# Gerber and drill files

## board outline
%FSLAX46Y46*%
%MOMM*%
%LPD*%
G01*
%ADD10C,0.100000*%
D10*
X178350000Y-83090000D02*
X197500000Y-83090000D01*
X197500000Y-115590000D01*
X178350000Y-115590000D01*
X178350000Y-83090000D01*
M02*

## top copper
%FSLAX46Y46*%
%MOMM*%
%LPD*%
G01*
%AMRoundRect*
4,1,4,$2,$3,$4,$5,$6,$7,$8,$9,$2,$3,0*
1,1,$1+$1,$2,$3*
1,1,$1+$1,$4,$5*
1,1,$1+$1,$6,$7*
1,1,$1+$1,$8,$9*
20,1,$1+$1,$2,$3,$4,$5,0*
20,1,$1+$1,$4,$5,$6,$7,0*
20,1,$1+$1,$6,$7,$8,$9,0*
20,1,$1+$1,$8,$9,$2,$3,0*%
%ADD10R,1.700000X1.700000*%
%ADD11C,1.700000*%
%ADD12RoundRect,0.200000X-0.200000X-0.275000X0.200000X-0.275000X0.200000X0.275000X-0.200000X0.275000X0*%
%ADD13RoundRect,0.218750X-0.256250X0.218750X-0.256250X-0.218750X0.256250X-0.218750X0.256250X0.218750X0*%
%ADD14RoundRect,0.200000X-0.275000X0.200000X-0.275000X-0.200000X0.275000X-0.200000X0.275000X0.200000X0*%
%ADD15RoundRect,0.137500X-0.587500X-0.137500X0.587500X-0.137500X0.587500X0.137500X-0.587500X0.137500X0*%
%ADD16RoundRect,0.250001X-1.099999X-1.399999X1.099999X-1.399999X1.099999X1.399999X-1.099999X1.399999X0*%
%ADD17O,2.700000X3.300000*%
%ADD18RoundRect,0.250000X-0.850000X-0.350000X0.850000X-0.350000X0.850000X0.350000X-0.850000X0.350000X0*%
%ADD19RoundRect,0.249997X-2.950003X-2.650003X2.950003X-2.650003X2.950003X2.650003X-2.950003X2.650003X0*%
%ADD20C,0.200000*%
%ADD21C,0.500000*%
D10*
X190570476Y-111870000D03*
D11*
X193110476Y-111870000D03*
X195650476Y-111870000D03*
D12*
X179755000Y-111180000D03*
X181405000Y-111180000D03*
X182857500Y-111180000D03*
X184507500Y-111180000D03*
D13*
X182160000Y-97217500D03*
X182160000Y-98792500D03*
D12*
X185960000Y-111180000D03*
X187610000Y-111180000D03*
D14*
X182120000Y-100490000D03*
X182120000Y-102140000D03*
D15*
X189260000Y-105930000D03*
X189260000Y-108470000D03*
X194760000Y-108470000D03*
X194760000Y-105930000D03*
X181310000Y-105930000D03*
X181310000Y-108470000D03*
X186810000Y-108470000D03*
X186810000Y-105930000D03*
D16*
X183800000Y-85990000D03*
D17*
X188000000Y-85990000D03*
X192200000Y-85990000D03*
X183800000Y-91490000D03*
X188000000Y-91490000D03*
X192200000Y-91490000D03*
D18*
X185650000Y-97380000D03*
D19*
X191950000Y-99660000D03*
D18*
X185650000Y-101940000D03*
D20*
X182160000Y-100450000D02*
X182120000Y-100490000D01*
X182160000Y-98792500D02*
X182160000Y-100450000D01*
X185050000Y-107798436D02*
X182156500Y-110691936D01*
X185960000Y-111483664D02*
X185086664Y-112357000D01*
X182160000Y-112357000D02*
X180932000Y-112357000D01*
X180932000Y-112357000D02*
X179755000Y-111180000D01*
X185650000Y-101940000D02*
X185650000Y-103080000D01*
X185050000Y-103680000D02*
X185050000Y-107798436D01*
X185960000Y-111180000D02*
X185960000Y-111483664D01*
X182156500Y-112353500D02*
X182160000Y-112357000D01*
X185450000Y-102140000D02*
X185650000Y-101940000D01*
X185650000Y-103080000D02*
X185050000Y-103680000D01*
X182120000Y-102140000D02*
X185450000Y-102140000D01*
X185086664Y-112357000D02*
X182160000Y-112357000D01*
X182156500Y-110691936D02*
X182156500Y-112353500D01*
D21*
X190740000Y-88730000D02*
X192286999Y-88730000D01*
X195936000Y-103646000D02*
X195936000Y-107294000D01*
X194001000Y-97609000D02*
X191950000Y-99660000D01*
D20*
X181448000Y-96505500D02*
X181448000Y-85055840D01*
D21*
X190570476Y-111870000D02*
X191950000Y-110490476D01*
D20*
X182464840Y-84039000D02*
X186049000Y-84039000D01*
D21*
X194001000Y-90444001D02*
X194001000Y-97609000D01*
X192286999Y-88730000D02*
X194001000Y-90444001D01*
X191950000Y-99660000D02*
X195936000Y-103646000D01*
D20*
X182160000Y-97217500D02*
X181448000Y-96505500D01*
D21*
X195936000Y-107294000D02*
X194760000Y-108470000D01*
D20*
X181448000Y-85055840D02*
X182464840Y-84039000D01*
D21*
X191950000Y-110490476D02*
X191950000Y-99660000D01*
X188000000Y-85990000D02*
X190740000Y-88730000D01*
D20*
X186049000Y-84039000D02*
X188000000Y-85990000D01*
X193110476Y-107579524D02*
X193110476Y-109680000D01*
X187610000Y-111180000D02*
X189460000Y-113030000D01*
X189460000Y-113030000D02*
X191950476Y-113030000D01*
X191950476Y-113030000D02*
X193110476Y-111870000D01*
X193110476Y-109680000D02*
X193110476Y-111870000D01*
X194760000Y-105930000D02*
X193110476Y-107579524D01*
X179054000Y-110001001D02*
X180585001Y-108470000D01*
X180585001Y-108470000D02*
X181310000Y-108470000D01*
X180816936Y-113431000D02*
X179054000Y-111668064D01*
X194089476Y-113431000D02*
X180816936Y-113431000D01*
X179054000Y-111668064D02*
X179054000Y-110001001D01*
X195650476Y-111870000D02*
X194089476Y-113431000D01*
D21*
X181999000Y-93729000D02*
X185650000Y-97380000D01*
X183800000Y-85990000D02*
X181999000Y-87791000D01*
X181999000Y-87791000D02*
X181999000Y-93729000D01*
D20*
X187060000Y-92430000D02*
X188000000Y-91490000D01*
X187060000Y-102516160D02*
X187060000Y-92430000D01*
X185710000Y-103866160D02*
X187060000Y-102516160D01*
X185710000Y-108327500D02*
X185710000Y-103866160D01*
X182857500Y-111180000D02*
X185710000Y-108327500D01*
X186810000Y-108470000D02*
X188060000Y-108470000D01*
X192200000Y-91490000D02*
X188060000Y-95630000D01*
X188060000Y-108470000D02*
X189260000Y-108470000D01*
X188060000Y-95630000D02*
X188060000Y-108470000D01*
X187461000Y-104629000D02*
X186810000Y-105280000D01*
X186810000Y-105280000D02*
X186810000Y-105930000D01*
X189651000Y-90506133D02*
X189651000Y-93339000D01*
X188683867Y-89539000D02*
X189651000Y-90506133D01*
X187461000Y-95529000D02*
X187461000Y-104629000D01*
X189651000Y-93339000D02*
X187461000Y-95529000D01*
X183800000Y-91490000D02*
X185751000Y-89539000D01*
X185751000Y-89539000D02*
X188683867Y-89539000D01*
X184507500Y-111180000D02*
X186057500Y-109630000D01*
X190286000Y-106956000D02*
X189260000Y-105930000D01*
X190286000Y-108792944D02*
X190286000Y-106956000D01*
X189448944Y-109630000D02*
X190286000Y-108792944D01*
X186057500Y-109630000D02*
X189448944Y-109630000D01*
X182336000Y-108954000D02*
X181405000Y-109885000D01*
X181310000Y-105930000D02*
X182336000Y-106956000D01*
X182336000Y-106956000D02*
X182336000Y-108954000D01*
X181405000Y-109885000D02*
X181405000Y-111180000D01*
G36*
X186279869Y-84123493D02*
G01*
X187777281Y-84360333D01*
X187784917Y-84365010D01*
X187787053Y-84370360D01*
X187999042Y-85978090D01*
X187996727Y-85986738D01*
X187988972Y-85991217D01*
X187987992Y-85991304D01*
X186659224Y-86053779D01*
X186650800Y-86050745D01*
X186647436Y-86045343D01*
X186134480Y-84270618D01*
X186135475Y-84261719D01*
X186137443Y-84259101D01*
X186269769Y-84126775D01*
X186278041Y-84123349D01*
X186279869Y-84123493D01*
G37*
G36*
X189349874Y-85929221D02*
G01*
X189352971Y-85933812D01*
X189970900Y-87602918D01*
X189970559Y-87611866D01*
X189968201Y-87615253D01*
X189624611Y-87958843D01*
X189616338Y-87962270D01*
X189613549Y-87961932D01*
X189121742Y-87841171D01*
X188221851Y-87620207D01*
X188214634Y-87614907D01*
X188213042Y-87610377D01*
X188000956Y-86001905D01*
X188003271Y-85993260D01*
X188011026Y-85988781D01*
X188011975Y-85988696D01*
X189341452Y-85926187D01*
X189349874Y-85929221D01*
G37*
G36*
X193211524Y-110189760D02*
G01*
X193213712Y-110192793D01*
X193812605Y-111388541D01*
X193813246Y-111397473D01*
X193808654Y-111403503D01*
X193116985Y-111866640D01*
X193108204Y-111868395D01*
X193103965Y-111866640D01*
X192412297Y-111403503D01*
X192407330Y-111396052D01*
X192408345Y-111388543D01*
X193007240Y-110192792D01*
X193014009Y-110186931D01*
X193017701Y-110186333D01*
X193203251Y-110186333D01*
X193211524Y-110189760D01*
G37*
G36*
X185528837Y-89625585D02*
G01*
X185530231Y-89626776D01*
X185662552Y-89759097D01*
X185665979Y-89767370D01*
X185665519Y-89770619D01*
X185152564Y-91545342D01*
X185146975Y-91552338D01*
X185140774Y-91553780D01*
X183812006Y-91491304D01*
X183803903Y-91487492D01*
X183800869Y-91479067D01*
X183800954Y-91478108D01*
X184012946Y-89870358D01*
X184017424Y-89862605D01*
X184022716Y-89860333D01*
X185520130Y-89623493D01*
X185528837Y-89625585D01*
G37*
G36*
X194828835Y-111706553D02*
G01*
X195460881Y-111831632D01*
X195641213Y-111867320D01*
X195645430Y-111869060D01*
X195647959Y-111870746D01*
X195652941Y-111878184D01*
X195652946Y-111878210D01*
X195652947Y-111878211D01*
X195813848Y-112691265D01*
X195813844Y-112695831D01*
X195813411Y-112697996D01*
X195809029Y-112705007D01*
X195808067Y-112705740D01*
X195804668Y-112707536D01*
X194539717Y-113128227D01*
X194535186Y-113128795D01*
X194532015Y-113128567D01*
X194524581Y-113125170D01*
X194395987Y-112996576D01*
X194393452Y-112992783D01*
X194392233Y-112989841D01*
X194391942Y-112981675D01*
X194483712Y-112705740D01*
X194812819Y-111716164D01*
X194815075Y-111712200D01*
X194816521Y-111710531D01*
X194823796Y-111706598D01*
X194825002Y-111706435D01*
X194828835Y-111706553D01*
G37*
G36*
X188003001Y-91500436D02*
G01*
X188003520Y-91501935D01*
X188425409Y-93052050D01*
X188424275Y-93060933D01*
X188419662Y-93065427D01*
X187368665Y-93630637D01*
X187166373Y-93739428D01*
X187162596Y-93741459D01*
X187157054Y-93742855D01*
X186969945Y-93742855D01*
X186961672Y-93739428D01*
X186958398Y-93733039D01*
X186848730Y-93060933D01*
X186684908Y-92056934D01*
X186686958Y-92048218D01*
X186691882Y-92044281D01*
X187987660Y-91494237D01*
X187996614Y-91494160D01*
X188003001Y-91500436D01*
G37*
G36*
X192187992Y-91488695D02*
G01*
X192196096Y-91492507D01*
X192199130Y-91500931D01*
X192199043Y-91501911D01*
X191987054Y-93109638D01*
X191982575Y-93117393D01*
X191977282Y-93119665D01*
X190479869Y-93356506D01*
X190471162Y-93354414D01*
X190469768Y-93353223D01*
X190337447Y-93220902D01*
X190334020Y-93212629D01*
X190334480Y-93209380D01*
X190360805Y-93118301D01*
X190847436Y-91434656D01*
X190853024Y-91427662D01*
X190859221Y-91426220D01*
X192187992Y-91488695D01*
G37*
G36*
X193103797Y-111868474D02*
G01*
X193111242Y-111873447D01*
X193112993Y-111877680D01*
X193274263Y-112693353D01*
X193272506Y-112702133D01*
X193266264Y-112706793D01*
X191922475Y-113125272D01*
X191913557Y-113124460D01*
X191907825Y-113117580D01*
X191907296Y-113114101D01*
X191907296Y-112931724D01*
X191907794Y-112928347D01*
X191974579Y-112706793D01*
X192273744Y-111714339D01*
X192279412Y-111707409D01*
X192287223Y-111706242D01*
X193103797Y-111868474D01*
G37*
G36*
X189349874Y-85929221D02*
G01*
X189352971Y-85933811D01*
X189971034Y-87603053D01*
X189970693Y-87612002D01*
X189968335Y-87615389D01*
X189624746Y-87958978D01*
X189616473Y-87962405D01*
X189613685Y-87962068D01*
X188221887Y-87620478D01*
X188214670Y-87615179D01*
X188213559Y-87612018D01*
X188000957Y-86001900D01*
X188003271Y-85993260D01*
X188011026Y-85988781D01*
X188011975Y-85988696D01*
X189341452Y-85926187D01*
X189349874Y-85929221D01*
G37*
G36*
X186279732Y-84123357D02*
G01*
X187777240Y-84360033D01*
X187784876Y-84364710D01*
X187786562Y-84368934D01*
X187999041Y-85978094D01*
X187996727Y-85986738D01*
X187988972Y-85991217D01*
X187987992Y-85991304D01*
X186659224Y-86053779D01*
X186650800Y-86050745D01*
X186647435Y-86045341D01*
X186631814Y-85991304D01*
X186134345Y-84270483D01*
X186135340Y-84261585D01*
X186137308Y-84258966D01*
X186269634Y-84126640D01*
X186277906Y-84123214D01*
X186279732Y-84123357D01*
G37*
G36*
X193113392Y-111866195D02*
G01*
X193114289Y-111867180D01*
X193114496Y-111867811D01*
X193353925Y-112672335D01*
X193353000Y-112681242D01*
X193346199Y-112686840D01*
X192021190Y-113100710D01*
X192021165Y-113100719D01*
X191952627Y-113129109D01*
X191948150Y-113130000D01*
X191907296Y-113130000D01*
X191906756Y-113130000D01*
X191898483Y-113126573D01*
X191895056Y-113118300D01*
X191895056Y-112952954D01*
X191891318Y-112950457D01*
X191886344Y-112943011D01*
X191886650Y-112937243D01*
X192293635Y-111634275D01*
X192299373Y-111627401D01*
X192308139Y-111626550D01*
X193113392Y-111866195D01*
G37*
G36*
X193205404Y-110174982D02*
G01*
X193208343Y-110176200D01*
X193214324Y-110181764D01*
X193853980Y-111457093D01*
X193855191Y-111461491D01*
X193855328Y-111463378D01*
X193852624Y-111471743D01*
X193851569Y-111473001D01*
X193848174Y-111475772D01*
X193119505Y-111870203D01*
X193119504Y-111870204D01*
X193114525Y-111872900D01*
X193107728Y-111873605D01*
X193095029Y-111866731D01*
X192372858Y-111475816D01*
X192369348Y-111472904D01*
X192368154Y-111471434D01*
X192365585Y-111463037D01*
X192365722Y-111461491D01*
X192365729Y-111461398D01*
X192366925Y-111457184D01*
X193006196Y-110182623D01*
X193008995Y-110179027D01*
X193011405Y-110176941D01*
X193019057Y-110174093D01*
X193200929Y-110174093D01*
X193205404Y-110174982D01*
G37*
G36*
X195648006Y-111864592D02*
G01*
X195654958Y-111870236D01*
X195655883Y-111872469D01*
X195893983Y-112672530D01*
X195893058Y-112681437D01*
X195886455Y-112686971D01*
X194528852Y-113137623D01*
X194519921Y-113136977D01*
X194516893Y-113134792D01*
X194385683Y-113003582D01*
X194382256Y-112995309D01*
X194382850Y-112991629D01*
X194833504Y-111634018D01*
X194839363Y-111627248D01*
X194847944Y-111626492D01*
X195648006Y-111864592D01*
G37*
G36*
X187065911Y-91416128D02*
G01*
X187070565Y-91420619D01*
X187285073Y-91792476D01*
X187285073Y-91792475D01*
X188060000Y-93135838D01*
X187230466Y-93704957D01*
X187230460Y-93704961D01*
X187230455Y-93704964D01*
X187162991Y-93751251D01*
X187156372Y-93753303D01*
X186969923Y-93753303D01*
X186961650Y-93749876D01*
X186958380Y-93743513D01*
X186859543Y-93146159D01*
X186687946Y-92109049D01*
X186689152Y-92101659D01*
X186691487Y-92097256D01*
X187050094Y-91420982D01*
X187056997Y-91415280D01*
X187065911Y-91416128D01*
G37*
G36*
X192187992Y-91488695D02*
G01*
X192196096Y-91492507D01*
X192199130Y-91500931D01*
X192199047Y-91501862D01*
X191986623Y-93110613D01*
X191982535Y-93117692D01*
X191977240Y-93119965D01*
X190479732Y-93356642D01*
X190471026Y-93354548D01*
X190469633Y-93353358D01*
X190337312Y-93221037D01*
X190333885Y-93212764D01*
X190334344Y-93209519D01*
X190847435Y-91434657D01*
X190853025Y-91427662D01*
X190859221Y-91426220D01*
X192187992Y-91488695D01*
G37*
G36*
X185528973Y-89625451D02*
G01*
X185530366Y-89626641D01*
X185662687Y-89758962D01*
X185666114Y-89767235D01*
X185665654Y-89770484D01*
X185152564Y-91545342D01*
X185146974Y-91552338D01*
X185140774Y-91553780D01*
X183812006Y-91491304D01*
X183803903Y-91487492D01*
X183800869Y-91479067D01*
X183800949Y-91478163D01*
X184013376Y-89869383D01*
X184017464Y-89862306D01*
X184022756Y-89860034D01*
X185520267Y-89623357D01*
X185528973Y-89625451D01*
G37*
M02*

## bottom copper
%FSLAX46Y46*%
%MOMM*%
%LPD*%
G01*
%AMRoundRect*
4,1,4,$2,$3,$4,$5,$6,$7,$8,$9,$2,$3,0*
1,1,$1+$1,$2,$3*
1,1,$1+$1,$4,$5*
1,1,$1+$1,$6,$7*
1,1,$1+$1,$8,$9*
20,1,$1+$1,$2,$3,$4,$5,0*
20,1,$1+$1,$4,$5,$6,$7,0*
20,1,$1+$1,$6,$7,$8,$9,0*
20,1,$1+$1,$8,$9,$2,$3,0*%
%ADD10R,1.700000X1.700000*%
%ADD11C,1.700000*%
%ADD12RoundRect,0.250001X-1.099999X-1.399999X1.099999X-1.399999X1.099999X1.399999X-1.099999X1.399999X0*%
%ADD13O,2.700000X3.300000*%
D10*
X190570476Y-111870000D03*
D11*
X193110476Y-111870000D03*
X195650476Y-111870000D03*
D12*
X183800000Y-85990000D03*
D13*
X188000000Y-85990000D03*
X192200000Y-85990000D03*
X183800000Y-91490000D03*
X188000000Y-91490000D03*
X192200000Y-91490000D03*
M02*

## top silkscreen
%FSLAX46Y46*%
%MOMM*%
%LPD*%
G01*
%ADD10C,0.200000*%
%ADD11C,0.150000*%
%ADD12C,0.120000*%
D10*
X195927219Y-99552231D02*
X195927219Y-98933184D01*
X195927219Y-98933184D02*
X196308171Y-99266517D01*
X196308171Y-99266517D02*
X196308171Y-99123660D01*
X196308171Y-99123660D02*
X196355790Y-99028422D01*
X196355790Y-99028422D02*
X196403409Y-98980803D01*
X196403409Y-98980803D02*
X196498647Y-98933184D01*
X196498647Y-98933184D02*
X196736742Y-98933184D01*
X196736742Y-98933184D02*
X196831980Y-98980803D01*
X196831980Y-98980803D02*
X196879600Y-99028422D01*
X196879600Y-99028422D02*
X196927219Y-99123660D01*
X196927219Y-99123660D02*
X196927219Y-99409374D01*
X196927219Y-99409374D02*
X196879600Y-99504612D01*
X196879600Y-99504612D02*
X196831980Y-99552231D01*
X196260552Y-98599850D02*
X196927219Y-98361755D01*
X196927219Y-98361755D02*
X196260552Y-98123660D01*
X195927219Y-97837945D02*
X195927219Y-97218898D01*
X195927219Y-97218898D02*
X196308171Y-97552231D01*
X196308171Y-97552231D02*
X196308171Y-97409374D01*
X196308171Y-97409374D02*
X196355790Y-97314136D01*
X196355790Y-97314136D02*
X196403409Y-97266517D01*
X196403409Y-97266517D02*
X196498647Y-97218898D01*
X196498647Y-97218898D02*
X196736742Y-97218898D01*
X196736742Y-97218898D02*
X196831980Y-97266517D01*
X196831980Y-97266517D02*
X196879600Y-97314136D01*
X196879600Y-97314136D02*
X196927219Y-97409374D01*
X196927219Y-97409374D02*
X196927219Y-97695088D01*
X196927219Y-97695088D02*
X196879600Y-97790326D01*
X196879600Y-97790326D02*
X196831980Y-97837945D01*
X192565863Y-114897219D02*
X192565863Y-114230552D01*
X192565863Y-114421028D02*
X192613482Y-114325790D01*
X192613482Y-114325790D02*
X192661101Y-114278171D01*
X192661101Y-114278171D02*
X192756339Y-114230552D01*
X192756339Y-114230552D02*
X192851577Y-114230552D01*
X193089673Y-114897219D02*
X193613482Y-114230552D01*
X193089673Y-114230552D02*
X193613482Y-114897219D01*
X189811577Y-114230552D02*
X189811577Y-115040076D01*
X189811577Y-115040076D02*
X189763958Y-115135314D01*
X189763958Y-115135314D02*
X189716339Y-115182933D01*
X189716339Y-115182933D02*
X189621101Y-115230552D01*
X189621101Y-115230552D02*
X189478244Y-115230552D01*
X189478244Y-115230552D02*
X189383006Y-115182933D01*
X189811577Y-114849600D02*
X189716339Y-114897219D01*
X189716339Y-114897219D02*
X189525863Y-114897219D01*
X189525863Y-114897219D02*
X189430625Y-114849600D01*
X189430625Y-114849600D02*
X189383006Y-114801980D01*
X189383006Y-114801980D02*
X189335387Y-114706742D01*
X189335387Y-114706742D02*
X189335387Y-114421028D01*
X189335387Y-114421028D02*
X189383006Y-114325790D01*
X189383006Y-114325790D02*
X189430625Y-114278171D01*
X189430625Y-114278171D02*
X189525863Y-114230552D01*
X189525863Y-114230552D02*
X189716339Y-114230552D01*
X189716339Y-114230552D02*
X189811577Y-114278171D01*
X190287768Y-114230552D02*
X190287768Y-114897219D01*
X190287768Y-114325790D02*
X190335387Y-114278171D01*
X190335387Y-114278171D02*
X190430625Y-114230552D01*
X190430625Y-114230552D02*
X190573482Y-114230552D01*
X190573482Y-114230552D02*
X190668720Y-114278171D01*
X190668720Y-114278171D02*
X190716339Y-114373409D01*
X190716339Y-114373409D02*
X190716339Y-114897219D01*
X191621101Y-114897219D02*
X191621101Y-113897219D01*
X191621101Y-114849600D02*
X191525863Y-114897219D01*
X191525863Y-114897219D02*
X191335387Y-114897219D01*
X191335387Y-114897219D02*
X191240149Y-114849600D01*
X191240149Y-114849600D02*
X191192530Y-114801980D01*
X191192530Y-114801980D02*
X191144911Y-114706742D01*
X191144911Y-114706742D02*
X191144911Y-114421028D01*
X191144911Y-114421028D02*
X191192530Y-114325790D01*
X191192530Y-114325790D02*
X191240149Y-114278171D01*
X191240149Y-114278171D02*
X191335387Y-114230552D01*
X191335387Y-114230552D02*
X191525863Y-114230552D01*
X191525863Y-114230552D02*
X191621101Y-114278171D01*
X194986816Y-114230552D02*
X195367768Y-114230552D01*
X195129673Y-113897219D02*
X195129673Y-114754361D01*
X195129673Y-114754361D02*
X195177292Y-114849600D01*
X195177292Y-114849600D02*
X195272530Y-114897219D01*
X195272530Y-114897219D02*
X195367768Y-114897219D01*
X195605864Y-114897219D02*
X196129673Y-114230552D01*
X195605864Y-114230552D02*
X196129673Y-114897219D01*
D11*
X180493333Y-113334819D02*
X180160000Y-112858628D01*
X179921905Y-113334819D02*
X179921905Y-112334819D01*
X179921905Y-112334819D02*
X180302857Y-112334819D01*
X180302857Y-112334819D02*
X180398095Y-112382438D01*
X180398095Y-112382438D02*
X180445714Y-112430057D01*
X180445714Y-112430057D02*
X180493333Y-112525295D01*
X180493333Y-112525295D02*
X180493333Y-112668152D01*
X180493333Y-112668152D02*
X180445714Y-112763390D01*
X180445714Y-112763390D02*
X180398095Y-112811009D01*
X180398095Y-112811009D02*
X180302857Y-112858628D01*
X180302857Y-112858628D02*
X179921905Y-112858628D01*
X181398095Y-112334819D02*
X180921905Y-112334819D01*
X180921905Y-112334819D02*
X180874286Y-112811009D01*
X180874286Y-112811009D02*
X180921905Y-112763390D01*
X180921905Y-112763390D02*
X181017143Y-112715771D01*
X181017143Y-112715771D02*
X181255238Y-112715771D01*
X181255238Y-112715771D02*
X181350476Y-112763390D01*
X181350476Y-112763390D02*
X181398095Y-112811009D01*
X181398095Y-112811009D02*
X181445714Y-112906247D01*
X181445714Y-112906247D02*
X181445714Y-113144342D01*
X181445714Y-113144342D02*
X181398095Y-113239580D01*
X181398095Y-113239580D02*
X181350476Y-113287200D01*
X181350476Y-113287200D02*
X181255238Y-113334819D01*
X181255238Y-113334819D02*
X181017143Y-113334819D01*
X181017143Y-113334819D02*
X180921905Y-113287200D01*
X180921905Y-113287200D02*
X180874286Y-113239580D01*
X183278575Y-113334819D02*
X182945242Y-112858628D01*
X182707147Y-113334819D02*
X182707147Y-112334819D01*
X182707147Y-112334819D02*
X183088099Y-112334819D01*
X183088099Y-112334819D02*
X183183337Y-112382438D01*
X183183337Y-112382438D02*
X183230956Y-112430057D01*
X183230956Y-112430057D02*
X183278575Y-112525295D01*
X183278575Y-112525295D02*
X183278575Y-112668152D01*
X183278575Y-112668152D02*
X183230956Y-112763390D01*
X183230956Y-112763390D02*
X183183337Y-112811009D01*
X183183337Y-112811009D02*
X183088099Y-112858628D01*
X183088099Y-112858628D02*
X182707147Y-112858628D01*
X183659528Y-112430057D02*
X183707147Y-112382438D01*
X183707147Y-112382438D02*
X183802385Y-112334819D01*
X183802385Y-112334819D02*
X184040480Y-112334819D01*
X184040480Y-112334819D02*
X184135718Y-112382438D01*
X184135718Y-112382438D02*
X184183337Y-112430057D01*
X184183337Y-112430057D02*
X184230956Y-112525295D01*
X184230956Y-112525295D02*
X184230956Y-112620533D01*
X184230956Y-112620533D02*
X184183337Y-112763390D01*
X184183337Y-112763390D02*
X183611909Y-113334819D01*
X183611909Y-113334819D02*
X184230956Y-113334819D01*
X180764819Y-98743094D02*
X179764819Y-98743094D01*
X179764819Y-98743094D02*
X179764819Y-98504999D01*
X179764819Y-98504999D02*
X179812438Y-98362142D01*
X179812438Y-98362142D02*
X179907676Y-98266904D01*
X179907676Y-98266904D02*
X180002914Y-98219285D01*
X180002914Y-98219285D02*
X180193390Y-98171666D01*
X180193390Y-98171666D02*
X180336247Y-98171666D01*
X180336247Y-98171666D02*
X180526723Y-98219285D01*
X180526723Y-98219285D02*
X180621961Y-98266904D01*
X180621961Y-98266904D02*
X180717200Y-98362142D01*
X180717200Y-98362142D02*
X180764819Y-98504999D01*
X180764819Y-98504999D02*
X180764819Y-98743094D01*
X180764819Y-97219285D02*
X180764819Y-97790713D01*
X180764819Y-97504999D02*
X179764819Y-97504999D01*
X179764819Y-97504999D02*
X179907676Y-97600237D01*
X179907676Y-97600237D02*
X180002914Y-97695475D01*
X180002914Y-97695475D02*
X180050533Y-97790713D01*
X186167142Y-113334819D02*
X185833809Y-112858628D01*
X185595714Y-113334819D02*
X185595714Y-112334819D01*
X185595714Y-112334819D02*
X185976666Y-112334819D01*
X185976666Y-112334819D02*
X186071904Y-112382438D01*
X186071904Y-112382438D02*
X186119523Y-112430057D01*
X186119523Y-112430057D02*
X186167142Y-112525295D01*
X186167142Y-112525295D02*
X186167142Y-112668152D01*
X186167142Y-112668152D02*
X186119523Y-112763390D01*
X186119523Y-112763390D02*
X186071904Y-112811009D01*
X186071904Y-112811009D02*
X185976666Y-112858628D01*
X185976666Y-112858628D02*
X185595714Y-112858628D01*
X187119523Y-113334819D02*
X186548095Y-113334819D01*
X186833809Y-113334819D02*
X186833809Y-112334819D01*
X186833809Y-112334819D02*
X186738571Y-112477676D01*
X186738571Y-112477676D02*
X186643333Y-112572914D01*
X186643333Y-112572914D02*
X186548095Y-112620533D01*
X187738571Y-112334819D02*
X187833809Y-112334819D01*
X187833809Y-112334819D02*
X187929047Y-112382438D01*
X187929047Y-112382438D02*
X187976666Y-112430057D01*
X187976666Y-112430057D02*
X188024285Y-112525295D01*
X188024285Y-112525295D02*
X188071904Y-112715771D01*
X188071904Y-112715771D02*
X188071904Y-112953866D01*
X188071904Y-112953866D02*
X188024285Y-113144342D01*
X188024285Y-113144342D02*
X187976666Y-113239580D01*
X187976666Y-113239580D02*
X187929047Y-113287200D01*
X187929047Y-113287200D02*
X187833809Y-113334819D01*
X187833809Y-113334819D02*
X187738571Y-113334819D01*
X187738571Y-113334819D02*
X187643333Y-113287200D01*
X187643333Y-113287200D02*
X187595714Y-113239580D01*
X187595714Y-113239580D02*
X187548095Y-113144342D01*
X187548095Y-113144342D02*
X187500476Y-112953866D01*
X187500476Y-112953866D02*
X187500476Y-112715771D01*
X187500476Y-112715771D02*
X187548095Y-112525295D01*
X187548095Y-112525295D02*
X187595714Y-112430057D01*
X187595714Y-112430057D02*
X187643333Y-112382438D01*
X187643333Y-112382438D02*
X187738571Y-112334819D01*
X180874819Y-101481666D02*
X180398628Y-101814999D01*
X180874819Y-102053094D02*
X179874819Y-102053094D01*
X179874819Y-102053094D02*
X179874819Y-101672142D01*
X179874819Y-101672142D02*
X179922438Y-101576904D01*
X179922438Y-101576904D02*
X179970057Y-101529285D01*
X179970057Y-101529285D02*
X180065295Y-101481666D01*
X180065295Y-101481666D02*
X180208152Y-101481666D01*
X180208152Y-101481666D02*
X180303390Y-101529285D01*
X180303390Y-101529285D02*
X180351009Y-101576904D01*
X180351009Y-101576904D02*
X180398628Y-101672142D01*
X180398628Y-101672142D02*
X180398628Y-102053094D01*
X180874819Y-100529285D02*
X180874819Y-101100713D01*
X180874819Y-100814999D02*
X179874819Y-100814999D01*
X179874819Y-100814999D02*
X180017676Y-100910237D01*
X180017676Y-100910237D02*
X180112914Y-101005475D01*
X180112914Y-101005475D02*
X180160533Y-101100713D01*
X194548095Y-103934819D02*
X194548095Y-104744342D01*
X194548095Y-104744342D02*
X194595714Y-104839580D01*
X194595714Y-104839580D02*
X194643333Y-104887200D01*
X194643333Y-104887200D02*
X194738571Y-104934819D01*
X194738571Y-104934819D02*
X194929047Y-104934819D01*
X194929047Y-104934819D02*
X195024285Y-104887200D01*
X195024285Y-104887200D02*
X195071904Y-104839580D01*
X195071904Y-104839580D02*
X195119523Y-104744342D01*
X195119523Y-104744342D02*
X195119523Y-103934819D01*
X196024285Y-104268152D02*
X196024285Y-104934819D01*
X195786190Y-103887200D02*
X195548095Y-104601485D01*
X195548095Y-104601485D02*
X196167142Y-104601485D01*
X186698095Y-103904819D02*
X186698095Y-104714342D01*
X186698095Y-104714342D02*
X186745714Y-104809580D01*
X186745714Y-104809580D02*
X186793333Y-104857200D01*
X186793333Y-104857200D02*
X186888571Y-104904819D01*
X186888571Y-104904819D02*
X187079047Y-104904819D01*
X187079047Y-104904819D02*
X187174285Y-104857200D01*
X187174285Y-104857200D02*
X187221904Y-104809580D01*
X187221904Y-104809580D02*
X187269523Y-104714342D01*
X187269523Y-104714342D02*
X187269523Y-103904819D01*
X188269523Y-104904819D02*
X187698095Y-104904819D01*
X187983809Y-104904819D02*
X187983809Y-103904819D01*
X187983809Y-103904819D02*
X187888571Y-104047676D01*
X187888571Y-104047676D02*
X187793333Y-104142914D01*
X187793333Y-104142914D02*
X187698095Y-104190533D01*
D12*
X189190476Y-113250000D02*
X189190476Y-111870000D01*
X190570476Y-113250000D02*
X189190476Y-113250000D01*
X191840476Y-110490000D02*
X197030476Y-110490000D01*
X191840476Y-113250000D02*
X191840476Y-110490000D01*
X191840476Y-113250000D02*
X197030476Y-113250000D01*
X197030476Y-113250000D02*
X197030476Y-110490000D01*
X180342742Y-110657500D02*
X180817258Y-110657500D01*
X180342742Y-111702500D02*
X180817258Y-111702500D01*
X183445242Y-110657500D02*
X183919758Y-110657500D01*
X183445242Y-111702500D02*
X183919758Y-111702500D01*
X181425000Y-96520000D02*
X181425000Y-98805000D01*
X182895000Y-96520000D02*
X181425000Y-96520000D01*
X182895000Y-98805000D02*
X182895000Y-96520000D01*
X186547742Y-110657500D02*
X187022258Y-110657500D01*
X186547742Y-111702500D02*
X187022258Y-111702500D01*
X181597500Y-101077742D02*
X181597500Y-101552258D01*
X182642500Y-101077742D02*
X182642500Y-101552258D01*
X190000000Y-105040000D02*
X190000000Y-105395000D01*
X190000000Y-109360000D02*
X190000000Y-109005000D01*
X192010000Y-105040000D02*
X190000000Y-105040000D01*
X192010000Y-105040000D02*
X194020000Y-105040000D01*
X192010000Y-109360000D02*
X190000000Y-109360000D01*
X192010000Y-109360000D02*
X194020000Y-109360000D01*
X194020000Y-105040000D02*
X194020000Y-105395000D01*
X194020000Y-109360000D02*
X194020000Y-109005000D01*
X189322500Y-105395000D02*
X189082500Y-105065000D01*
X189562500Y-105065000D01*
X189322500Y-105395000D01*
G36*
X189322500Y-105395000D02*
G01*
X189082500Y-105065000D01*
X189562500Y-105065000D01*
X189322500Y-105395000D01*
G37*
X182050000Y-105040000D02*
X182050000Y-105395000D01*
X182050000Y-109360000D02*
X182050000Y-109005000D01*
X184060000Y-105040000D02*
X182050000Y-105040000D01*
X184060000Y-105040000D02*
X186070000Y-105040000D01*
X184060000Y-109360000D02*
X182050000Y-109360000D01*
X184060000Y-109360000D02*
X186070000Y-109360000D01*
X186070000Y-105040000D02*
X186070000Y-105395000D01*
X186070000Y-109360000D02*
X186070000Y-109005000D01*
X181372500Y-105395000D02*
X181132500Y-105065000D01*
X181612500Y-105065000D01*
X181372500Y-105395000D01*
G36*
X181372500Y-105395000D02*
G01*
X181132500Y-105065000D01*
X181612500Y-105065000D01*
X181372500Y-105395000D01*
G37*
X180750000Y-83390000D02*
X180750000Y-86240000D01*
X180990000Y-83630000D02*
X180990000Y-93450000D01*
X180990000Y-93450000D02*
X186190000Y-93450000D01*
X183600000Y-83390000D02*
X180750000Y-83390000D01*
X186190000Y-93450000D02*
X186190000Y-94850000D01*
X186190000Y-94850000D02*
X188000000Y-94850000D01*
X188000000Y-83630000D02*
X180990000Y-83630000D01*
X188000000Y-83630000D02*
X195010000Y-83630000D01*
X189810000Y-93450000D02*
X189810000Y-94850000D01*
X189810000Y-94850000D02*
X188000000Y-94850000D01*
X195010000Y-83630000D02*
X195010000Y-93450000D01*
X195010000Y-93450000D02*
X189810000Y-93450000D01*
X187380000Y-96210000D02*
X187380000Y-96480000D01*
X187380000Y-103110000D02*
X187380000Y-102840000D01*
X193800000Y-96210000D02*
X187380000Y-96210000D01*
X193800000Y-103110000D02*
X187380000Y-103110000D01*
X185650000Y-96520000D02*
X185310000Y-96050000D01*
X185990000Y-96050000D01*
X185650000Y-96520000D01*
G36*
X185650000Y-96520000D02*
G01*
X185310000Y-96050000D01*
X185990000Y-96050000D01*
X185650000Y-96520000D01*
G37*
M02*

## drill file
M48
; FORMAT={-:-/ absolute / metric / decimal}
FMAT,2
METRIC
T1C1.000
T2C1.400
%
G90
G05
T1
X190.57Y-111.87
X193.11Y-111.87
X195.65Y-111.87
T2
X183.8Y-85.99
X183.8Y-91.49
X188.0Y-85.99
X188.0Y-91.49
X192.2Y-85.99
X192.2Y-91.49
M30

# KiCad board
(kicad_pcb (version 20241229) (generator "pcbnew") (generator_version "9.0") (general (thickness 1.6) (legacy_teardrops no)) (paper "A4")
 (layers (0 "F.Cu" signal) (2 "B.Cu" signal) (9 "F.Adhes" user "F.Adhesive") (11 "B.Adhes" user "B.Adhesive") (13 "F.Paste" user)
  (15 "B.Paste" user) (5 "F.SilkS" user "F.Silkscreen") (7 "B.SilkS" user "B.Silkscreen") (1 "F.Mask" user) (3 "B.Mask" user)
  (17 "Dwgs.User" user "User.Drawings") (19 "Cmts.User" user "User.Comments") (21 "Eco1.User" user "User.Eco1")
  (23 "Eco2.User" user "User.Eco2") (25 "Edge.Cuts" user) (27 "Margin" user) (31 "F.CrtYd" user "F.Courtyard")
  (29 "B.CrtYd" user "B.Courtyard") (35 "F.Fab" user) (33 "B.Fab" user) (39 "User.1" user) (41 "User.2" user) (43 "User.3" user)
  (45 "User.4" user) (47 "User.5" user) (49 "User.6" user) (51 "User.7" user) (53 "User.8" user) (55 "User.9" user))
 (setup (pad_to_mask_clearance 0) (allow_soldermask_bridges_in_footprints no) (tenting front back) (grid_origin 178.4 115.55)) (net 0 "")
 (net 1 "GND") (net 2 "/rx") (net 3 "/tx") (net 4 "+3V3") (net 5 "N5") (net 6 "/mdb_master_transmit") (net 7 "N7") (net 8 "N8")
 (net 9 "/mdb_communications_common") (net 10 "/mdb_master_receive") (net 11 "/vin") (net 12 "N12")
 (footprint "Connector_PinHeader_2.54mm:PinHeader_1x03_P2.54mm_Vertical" (layer "F.Cu") (at 190.570476 111.87 90)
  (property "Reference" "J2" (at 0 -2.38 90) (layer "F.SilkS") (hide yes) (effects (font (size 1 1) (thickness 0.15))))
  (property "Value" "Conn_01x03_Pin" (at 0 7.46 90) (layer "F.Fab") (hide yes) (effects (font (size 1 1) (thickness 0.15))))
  (fp_line (start -1.38 -1.38) (end 0 -1.38) (stroke (width 0.12) (type solid)) (layer "F.SilkS"))
  (fp_line (start -1.38 0) (end -1.38 -1.38) (stroke (width 0.12) (type solid)) (layer "F.SilkS"))
  (fp_line (start 1.38 1.27) (end 1.38 6.46) (stroke (width 0.12) (type solid)) (layer "F.SilkS"))
  (fp_line (start -1.38 1.27) (end 1.38 1.27) (stroke (width 0.12) (type solid)) (layer "F.SilkS"))
  (fp_line (start -1.38 1.27) (end -1.38 6.46) (stroke (width 0.12) (type solid)) (layer "F.SilkS"))
  (fp_line (start -1.38 6.46) (end 1.38 6.46) (stroke (width 0.12) (type solid)) (layer "F.SilkS"))
  (pad "1" thru_hole rect (at 0 0 90) (size 1.7 1.7) (drill 1) (layers "*.Cu" "*.Mask") (remove_unused_layers no) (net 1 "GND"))
  (pad "2" thru_hole circle (at 0 2.54 90) (size 1.7 1.7) (drill 1) (layers "*.Cu" "*.Mask") (remove_unused_layers no) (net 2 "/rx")
   (teardrops (best_length_ratio 0.5) (max_length 1) (best_width_ratio 1) (max_width 2) (curved_edges no) (filter_ratio 0.9) (enabled yes)
    (allow_two_segments yes) (prefer_zone_connections yes)))
  (pad "3" thru_hole circle (at 0 5.08 90) (size 1.7 1.7) (drill 1) (layers "*.Cu" "*.Mask") (remove_unused_layers no) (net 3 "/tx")
   (teardrops (best_length_ratio 0.5) (max_length 1) (best_width_ratio 1) (max_width 2) (curved_edges no) (filter_ratio 0.9) (enabled yes)
    (allow_two_segments yes) (prefer_zone_connections yes))))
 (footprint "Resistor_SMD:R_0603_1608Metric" (layer "F.Cu") (at 180.58 111.18)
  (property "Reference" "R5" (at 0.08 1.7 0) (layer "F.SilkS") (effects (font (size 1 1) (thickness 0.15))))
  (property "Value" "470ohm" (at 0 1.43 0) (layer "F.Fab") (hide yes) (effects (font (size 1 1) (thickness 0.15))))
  (fp_line (start -0.237258 -0.5225) (end 0.237258 -0.5225) (stroke (width 0.12) (type solid)) (layer "F.SilkS"))
  (fp_line (start -0.237258 0.5225) (end 0.237258 0.5225) (stroke (width 0.12) (type solid)) (layer "F.SilkS"))
  (pad "1" smd roundrect (at -0.825 0) (size 0.8 0.95) (layers "F.Cu" "F.Mask" "F.Paste") (roundrect_rratio 0.25) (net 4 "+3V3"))
  (pad "2" smd roundrect (at 0.825 0) (size 0.8 0.95) (layers "F.Cu" "F.Mask" "F.Paste") (roundrect_rratio 0.25) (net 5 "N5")))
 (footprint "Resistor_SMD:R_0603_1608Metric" (layer "F.Cu") (at 183.6825 111.18)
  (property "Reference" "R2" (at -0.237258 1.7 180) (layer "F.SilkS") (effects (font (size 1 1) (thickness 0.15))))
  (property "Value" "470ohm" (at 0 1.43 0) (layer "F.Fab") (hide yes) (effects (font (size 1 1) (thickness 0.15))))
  (fp_line (start -0.237258 -0.5225) (end 0.237258 -0.5225) (stroke (width 0.12) (type solid)) (layer "F.SilkS"))
  (fp_line (start -0.237258 0.5225) (end 0.237258 0.5225) (stroke (width 0.12) (type solid)) (layer "F.SilkS"))
  (pad "1" smd roundrect (at -0.825 0) (size 0.8 0.95) (layers "F.Cu" "F.Mask" "F.Paste") (roundrect_rratio 0.25)
   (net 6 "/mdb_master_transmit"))
  (pad "2" smd roundrect (at 0.825 0) (size 0.8 0.95) (layers "F.Cu" "F.Mask" "F.Paste") (roundrect_rratio 0.25) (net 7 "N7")))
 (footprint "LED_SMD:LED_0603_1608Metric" (layer "F.Cu") (at 182.16 98.005 -90)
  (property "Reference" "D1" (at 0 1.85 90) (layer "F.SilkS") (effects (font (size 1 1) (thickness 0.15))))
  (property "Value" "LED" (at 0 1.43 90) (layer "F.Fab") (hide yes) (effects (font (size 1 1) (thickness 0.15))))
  (fp_line (start -1.485 0.735) (end 0.8 0.735) (stroke (width 0.12) (type solid)) (layer "F.SilkS"))
  (fp_line (start -1.485 -0.735) (end -1.485 0.735) (stroke (width 0.12) (type solid)) (layer "F.SilkS"))
  (fp_line (start 0.8 -0.735) (end -1.485 -0.735) (stroke (width 0.12) (type solid)) (layer "F.SilkS"))
  (pad "1" smd roundrect (at -0.7875 0 270) (size 0.875 0.95) (layers "F.Cu" "F.Mask" "F.Paste") (roundrect_rratio 0.25) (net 1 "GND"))
  (pad "2" smd roundrect (at 0.7875 0 270) (size 0.875 0.95) (layers "F.Cu" "F.Mask" "F.Paste") (roundrect_rratio 0.25) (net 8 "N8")))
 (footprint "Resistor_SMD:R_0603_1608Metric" (layer "F.Cu") (at 186.785 111.18)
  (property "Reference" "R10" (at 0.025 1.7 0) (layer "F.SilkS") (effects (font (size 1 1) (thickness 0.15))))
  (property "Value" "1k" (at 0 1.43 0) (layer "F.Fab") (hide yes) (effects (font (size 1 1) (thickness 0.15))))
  (fp_line (start -0.237258 -0.5225) (end 0.237258 -0.5225) (stroke (width 0.12) (type solid)) (layer "F.SilkS"))
  (fp_line (start -0.237258 0.5225) (end 0.237258 0.5225) (stroke (width 0.12) (type solid)) (layer "F.SilkS"))
  (pad "1" smd roundrect (at -0.825 0) (size 0.8 0.95) (layers "F.Cu" "F.Mask" "F.Paste") (roundrect_rratio 0.25) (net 4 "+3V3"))
  (pad "2" smd roundrect (at 0.825 0) (size 0.8 0.95) (layers "F.Cu" "F.Mask" "F.Paste") (roundrect_rratio 0.25) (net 2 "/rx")))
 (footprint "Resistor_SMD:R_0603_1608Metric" (layer "F.Cu") (at 182.12 101.315 -90)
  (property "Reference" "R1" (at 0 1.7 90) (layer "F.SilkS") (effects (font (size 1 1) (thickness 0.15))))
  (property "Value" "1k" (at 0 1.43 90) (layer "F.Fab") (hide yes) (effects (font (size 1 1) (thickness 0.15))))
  (fp_line (start -0.237258 0.5225) (end 0.237258 0.5225) (stroke (width 0.12) (type solid)) (layer "F.SilkS"))
  (fp_line (start -0.237258 -0.5225) (end 0.237258 -0.5225) (stroke (width 0.12) (type solid)) (layer "F.SilkS"))
  (pad "1" smd roundrect (at -0.825 0 270) (size 0.8 0.95) (layers "F.Cu" "F.Mask" "F.Paste") (roundrect_rratio 0.25) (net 8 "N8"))
  (pad "2" smd roundrect (at 0.825 0 270) (size 0.8 0.95) (layers "F.Cu" "F.Mask" "F.Paste") (roundrect_rratio 0.25) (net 4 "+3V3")))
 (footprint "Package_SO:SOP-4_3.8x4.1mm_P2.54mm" (layer "F.Cu") (at 192.01 107.2)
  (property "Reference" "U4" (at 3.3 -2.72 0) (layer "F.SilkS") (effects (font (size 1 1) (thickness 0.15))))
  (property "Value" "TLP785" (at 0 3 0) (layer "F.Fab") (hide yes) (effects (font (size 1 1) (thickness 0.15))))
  (fp_line (start -2.01 -2.16) (end -2.01 -1.805) (stroke (width 0.12) (type solid)) (layer "F.SilkS"))
  (fp_line (start -2.01 2.16) (end -2.01 1.805) (stroke (width 0.12) (type solid)) (layer "F.SilkS"))
  (fp_line (start 0 -2.16) (end -2.01 -2.16) (stroke (width 0.12) (type solid)) (layer "F.SilkS"))
  (fp_line (start 0 -2.16) (end 2.01 -2.16) (stroke (width 0.12) (type solid)) (layer "F.SilkS"))
  (fp_line (start 0 2.16) (end -2.01 2.16) (stroke (width 0.12) (type solid)) (layer "F.SilkS"))
  (fp_line (start 0 2.16) (end 2.01 2.16) (stroke (width 0.12) (type solid)) (layer "F.SilkS"))
  (fp_line (start 2.01 -2.16) (end 2.01 -1.805) (stroke (width 0.12) (type solid)) (layer "F.SilkS"))
  (fp_line (start 2.01 2.16) (end 2.01 1.805) (stroke (width 0.12) (type solid)) (layer "F.SilkS"))
  (fp_poly
   (pts (xy -2.6875 -1.805) (xy -2.9275 -2.135) (xy -2.4475 -2.135)) (stroke (width 0.12) (type solid)) (fill yes) (layer "F.SilkS"))
  (pad "1" smd roundrect (at -2.75 -1.27) (size 1.45 0.55) (layers "F.Cu" "F.Mask" "F.Paste") (roundrect_rratio 0.25) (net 7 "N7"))
  (pad "2" smd roundrect (at -2.75 1.27) (size 1.45 0.55) (layers "F.Cu" "F.Mask" "F.Paste") (roundrect_rratio 0.25)
   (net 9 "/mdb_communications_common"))
  (pad "3" smd roundrect (at 2.75 1.27) (size 1.45 0.55) (layers "F.Cu" "F.Mask" "F.Paste") (roundrect_rratio 0.25) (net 1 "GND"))
  (pad "4" smd roundrect (at 2.75 -1.27) (size 1.45 0.55) (layers "F.Cu" "F.Mask" "F.Paste") (roundrect_rratio 0.25) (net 2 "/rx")))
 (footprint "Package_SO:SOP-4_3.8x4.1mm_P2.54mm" (layer "F.Cu") (at 184.06 107.2)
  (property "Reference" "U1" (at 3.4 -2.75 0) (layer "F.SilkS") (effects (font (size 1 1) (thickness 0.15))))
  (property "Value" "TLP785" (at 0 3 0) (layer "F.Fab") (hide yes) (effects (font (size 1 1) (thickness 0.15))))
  (fp_line (start -2.01 -2.16) (end -2.01 -1.805) (stroke (width 0.12) (type solid)) (layer "F.SilkS"))
  (fp_line (start -2.01 2.16) (end -2.01 1.805) (stroke (width 0.12) (type solid)) (layer "F.SilkS"))
  (fp_line (start 0 -2.16) (end -2.01 -2.16) (stroke (width 0.12) (type solid)) (layer "F.SilkS"))
  (fp_line (start 0 -2.16) (end 2.01 -2.16) (stroke (width 0.12) (type solid)) (layer "F.SilkS"))
  (fp_line (start 0 2.16) (end -2.01 2.16) (stroke (width 0.12) (type solid)) (layer "F.SilkS"))
  (fp_line (start 0 2.16) (end 2.01 2.16) (stroke (width 0.12) (type solid)) (layer "F.SilkS"))
  (fp_line (start 2.01 -2.16) (end 2.01 -1.805) (stroke (width 0.12) (type solid)) (layer "F.SilkS"))
  (fp_line (start 2.01 2.16) (end 2.01 1.805) (stroke (width 0.12) (type solid)) (layer "F.SilkS"))
  (fp_poly
   (pts (xy -2.6875 -1.805) (xy -2.9275 -2.135) (xy -2.4475 -2.135)) (stroke (width 0.12) (type solid)) (fill yes) (layer "F.SilkS"))
  (pad "1" smd roundrect (at -2.75 -1.27) (size 1.45 0.55) (layers "F.Cu" "F.Mask" "F.Paste") (roundrect_rratio 0.25) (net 5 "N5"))
  (pad "2" smd roundrect (at -2.75 1.27) (size 1.45 0.55) (layers "F.Cu" "F.Mask" "F.Paste") (roundrect_rratio 0.25) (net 3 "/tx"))
  (pad "3" smd roundrect (at 2.75 1.27) (size 1.45 0.55) (layers "F.Cu" "F.Mask" "F.Paste") (roundrect_rratio 0.25)
   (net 9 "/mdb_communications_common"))
  (pad "4" smd roundrect (at 2.75 -1.27) (size 1.45 0.55) (layers "F.Cu" "F.Mask" "F.Paste") (roundrect_rratio 0.25)
   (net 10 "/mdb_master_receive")))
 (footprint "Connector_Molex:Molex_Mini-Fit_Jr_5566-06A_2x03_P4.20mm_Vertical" (layer "F.Cu") (at 183.8 85.99)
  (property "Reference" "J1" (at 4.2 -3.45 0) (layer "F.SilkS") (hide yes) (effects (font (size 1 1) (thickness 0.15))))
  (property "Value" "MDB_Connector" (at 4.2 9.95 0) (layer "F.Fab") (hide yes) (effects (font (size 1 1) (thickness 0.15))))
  (fp_line (start -3.05 -2.6) (end -3.05 0.25) (stroke (width 0.12) (type solid)) (layer "F.SilkS"))
  (fp_line (start -2.81 -2.36) (end -2.81 7.46) (stroke (width 0.12) (type solid)) (layer "F.SilkS"))
  (fp_line (start -2.81 7.46) (end 2.39 7.46) (stroke (width 0.12) (type solid)) (layer "F.SilkS"))
  (fp_line (start -0.2 -2.6) (end -3.05 -2.6) (stroke (width 0.12) (type solid)) (layer "F.SilkS"))
  (fp_line (start 2.39 7.46) (end 2.39 8.86) (stroke (width 0.12) (type solid)) (layer "F.SilkS"))
  (fp_line (start 2.39 8.86) (end 4.2 8.86) (stroke (width 0.12) (type solid)) (layer "F.SilkS"))
  (fp_line (start 4.2 -2.36) (end -2.81 -2.36) (stroke (width 0.12) (type solid)) (layer "F.SilkS"))
  (fp_line (start 4.2 -2.36) (end 11.21 -2.36) (stroke (width 0.12) (type solid)) (layer "F.SilkS"))
  (fp_line (start 6.01 7.46) (end 6.01 8.86) (stroke (width 0.12) (type solid)) (layer "F.SilkS"))
  (fp_line (start 6.01 8.86) (end 4.2 8.86) (stroke (width 0.12) (type solid)) (layer "F.SilkS"))
  (fp_line (start 11.21 -2.36) (end 11.21 7.46) (stroke (width 0.12) (type solid)) (layer "F.SilkS"))
  (fp_line (start 11.21 7.46) (end 6.01 7.46) (stroke (width 0.12) (type solid)) (layer "F.SilkS"))
  (pad "1" thru_hole roundrect (at 0 0) (size 2.7 3.3) (drill 1.4) (layers "*.Cu" "*.Mask") (remove_unused_layers no)
   (roundrect_rratio 0.092593) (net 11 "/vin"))
  (pad "2" thru_hole oval (at 4.2 0) (size 2.7 3.3) (drill 1.4) (layers "*.Cu" "*.Mask") (remove_unused_layers no) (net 1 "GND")
   (teardrops (best_length_ratio 0.5) (max_length 1) (best_width_ratio 1) (max_width 2) (curved_edges no) (filter_ratio 0.9) (enabled yes)
    (allow_two_segments yes) (prefer_zone_connections yes)))
  (pad "3" thru_hole oval (at 8.4 0) (size 2.7 3.3) (drill 1.4) (layers "*.Cu" "*.Mask") (remove_unused_layers no) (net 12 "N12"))
  (pad "4" thru_hole oval (at 0 5.5) (size 2.7 3.3) (drill 1.4) (layers "*.Cu" "*.Mask") (remove_unused_layers no)
   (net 10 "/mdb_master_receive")
   (teardrops (best_length_ratio 0.5) (max_length 1) (best_width_ratio 1) (max_width 2) (curved_edges no) (filter_ratio 0.9) (enabled yes)
    (allow_two_segments yes) (prefer_zone_connections yes)))
  (pad "5" thru_hole oval (at 4.2 5.5) (size 2.7 3.3) (drill 1.4) (layers "*.Cu" "*.Mask") (remove_unused_layers no)
   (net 6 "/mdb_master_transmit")
   (teardrops (best_length_ratio 0.5) (max_length 1) (best_width_ratio 1) (max_width 2) (curved_edges no) (filter_ratio 0.9) (enabled yes)
    (allow_two_segments yes) (prefer_zone_connections yes)))
  (pad "6" thru_hole oval (at 8.4 5.5) (size 2.7 3.3) (drill 1.4) (layers "*.Cu" "*.Mask") (remove_unused_layers no)
   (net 9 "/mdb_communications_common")
   (teardrops (best_length_ratio 0.5) (max_length 1) (best_width_ratio 1) (max_width 2) (curved_edges no) (filter_ratio 0.9) (enabled yes)
    (allow_two_segments yes) (prefer_zone_connections yes))))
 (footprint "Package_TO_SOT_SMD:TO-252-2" (layer "F.Cu") (at 190.69 99.66)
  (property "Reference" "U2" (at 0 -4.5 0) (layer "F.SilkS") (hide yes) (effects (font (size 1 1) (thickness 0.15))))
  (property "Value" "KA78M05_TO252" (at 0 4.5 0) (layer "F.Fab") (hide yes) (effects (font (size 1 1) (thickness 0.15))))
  (fp_line (start -3.31 -3.45) (end -3.31 -3.18) (stroke (width 0.12) (type solid)) (layer "F.SilkS"))
  (fp_line (start -3.31 3.45) (end -3.31 3.18) (stroke (width 0.12) (type solid)) (layer "F.SilkS"))
  (fp_line (start 3.11 -3.45) (end -3.31 -3.45) (stroke (width 0.12) (type solid)) (layer "F.SilkS"))
  (fp_line (start 3.11 3.45) (end -3.31 3.45) (stroke (width 0.12) (type solid)) (layer "F.SilkS"))
  (fp_poly (pts (xy -5.04 -3.14) (xy -5.38 -3.61) (xy -4.7 -3.61)) (stroke (width 0.12) (type solid)) (fill yes) (layer "F.SilkS"))
  (pad "" smd roundrect (at -0.415 -1.525) (size 3.05 2.75) (layers "F.Paste") (roundrect_rratio 0.090909))
  (pad "" smd roundrect (at -0.415 1.525) (size 3.05 2.75) (layers "F.Paste") (roundrect_rratio 0.090909))
  (pad "" smd roundrect (at 2.935 -1.525) (size 3.05 2.75) (layers "F.Paste") (roundrect_rratio 0.090909))
  (pad "" smd roundrect (at 2.935 1.525) (size 3.05 2.75) (layers "F.Paste") (roundrect_rratio 0.090909))
  (pad "1" smd roundrect (at -5.04 -2.28) (size 2.2 1.2) (layers "F.Cu" "F.Mask" "F.Paste") (roundrect_rratio 0.208333) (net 11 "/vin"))
  (pad "2" smd roundrect (at 1.26 0) (size 6.4 5.8) (layers "F.Cu" "F.Mask") (roundrect_rratio 0.043103) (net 1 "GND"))
  (pad "3" smd roundrect (at -5.04 2.28) (size 2.2 1.2) (layers "F.Cu" "F.Mask" "F.Paste") (roundrect_rratio 0.208333) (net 4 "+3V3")))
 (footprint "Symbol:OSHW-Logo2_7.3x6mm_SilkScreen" (layer "B.Cu") (at 188 105.35 180)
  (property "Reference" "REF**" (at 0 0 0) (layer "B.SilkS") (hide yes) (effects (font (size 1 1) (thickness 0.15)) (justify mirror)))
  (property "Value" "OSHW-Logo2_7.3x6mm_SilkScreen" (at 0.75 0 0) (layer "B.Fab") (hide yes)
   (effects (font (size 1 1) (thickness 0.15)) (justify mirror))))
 (gr_rect (start 178.35 83.09) (end 197.5 115.59) (stroke (width 0.1) (type solid)) (fill no) (layer "Edge.Cuts"))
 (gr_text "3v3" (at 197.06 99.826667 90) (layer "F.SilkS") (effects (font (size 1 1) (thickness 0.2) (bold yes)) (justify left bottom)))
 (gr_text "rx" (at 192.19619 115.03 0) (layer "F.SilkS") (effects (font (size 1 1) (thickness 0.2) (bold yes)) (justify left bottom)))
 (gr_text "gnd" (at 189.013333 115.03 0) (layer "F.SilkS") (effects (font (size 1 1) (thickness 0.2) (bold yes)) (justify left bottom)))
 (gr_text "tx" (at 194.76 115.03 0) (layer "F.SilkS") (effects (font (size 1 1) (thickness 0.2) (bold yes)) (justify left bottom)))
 (segment (start 182.16 100.45) (end 182.12 100.49) (width 0.2) (layer "F.Cu") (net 8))
 (segment (start 182.16 98.7925) (end 182.16 100.45) (width 0.2) (layer "F.Cu") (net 8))
 (segment (start 185.05 107.798436) (end 182.1565 110.691936) (width 0.2) (layer "F.Cu") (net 4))
 (segment (start 185.96 111.483664) (end 185.086664 112.357) (width 0.2) (layer "F.Cu") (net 4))
 (segment (start 182.16 112.357) (end 180.932 112.357) (width 0.2) (layer "F.Cu") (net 4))
 (segment (start 180.932 112.357) (end 179.755 111.18) (width 0.2) (layer "F.Cu") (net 4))
 (segment (start 185.65 101.94) (end 185.65 103.08) (width 0.2) (layer "F.Cu") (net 4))
 (segment (start 185.05 103.68) (end 185.05 107.798436) (width 0.2) (layer "F.Cu") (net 4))
 (segment (start 185.96 111.18) (end 185.96 111.483664) (width 0.2) (layer "F.Cu") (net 4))
 (segment (start 182.1565 112.3535) (end 182.16 112.357) (width 0.2) (layer "F.Cu") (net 4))
 (segment (start 185.45 102.14) (end 185.65 101.94) (width 0.2) (layer "F.Cu") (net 4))
 (segment (start 185.65 103.08) (end 185.05 103.68) (width 0.2) (layer "F.Cu") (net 4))
 (segment (start 182.12 102.14) (end 185.45 102.14) (width 0.2) (layer "F.Cu") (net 4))
 (segment (start 185.086664 112.357) (end 182.16 112.357) (width 0.2) (layer "F.Cu") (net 4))
 (segment (start 182.1565 110.691936) (end 182.1565 112.3535) (width 0.2) (layer "F.Cu") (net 4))
 (segment (start 190.74 88.73) (end 192.286999 88.73) (width 0.5) (layer "F.Cu") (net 1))
 (segment (start 195.936 103.646) (end 195.936 107.294) (width 0.5) (layer "F.Cu") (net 1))
 (segment (start 194.001 97.609) (end 191.95 99.66) (width 0.5) (layer "F.Cu") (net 1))
 (segment (start 181.448 96.5055) (end 181.448 85.05584) (width 0.2) (layer "F.Cu") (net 1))
 (segment (start 190.570476 111.87) (end 191.95 110.490476) (width 0.5) (layer "F.Cu") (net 1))
 (segment (start 182.46484 84.039) (end 186.049 84.039) (width 0.2) (layer "F.Cu") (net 1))
 (segment (start 194.001 90.444001) (end 194.001 97.609) (width 0.5) (layer "F.Cu") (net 1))
 (segment (start 192.286999 88.73) (end 194.001 90.444001) (width 0.5) (layer "F.Cu") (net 1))
 (segment (start 191.95 99.66) (end 195.936 103.646) (width 0.5) (layer "F.Cu") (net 1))
 (segment (start 182.16 97.2175) (end 181.448 96.5055) (width 0.2) (layer "F.Cu") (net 1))
 (segment (start 195.936 107.294) (end 194.76 108.47) (width 0.5) (layer "F.Cu") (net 1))
 (segment (start 181.448 85.05584) (end 182.46484 84.039) (width 0.2) (layer "F.Cu") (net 1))
 (segment (start 191.95 110.490476) (end 191.95 99.66) (width 0.5) (layer "F.Cu") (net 1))
 (segment (start 188 85.99) (end 190.74 88.73) (width 0.5) (layer "F.Cu") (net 1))
 (segment (start 186.049 84.039) (end 188 85.99) (width 0.2) (layer "F.Cu") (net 1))
 (segment (start 193.110476 107.579524) (end 193.110476 109.68) (width 0.2) (layer "F.Cu") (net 2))
 (segment (start 187.61 111.18) (end 189.46 113.03) (width 0.2) (layer "F.Cu") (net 2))
 (segment (start 189.46 113.03) (end 191.950476 113.03) (width 0.2) (layer "F.Cu") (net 2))
 (segment (start 191.950476 113.03) (end 193.110476 111.87) (width 0.2) (layer "F.Cu") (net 2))
 (segment (start 193.110476 109.68) (end 193.110476 111.87) (width 0.2) (layer "F.Cu") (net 2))
 (segment (start 194.76 105.93) (end 193.110476 107.579524) (width 0.2) (layer "F.Cu") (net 2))
 (segment (start 179.054 110.001001) (end 180.585001 108.47) (width 0.2) (layer "F.Cu") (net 3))
 (segment (start 180.585001 108.47) (end 181.31 108.47) (width 0.2) (layer "F.Cu") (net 3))
 (segment (start 180.816936 113.431) (end 179.054 111.668064) (width 0.2) (layer "F.Cu") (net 3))
 (segment (start 194.089476 113.431) (end 180.816936 113.431) (width 0.2) (layer "F.Cu") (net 3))
 (segment (start 179.054 111.668064) (end 179.054 110.001001) (width 0.2) (layer "F.Cu") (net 3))
 (segment (start 195.650476 111.87) (end 194.089476 113.431) (width 0.2) (layer "F.Cu") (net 3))
 (segment (start 181.999 93.729) (end 185.65 97.38) (width 0.5) (layer "F.Cu") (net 11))
 (segment (start 183.8 85.99) (end 181.999 87.791) (width 0.5) (layer "F.Cu") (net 11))
 (segment (start 181.999 87.791) (end 181.999 93.729) (width 0.5) (layer "F.Cu") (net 11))
 (segment (start 187.06 92.43) (end 188 91.49) (width 0.2) (layer "F.Cu") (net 6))
 (segment (start 187.06 102.51616) (end 187.06 92.43) (width 0.2) (layer "F.Cu") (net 6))
 (segment (start 185.71 103.86616) (end 187.06 102.51616) (width 0.2) (layer "F.Cu") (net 6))
 (segment (start 185.71 108.3275) (end 185.71 103.86616) (width 0.2) (layer "F.Cu") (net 6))
 (segment (start 182.8575 111.18) (end 185.71 108.3275) (width 0.2) (layer "F.Cu") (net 6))
 (segment (start 186.81 108.47) (end 188.06 108.47) (width 0.2) (layer "F.Cu") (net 9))
 (segment (start 192.2 91.49) (end 188.06 95.63) (width 0.2) (layer "F.Cu") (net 9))
 (segment (start 188.06 108.47) (end 189.26 108.47) (width 0.2) (layer "F.Cu") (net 9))
 (segment (start 188.06 95.63) (end 188.06 108.47) (width 0.2) (layer "F.Cu") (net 9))
 (segment (start 187.461 104.629) (end 186.81 105.28) (width 0.2) (layer "F.Cu") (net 10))
 (segment (start 186.81 105.28) (end 186.81 105.93) (width 0.2) (layer "F.Cu") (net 10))
 (segment (start 189.651 90.506133) (end 189.651 93.339) (width 0.2) (layer "F.Cu") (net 10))
 (segment (start 188.683867 89.539) (end 189.651 90.506133) (width 0.2) (layer "F.Cu") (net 10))
 (segment (start 187.461 95.529) (end 187.461 104.629) (width 0.2) (layer "F.Cu") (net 10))
 (segment (start 189.651 93.339) (end 187.461 95.529) (width 0.2) (layer "F.Cu") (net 10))
 (segment (start 183.8 91.49) (end 185.751 89.539) (width 0.2) (layer "F.Cu") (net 10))
 (segment (start 185.751 89.539) (end 188.683867 89.539) (width 0.2) (layer "F.Cu") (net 10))
 (segment (start 184.5075 111.18) (end 186.0575 109.63) (width 0.2) (layer "F.Cu") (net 7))
 (segment (start 190.286 106.956) (end 189.26 105.93) (width 0.2) (layer "F.Cu") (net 7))
 (segment (start 190.286 108.792944) (end 190.286 106.956) (width 0.2) (layer "F.Cu") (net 7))
 (segment (start 189.448944 109.63) (end 190.286 108.792944) (width 0.2) (layer "F.Cu") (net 7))
 (segment (start 186.0575 109.63) (end 189.448944 109.63) (width 0.2) (layer "F.Cu") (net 7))
 (segment (start 182.336 108.954) (end 181.405 109.885) (width 0.2) (layer "F.Cu") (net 5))
 (segment (start 181.31 105.93) (end 182.336 106.956) (width 0.2) (layer "F.Cu") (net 5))
 (segment (start 182.336 106.956) (end 182.336 108.954) (width 0.2) (layer "F.Cu") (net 5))
 (segment (start 181.405 109.885) (end 181.405 111.18) (width 0.2) (layer "F.Cu") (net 5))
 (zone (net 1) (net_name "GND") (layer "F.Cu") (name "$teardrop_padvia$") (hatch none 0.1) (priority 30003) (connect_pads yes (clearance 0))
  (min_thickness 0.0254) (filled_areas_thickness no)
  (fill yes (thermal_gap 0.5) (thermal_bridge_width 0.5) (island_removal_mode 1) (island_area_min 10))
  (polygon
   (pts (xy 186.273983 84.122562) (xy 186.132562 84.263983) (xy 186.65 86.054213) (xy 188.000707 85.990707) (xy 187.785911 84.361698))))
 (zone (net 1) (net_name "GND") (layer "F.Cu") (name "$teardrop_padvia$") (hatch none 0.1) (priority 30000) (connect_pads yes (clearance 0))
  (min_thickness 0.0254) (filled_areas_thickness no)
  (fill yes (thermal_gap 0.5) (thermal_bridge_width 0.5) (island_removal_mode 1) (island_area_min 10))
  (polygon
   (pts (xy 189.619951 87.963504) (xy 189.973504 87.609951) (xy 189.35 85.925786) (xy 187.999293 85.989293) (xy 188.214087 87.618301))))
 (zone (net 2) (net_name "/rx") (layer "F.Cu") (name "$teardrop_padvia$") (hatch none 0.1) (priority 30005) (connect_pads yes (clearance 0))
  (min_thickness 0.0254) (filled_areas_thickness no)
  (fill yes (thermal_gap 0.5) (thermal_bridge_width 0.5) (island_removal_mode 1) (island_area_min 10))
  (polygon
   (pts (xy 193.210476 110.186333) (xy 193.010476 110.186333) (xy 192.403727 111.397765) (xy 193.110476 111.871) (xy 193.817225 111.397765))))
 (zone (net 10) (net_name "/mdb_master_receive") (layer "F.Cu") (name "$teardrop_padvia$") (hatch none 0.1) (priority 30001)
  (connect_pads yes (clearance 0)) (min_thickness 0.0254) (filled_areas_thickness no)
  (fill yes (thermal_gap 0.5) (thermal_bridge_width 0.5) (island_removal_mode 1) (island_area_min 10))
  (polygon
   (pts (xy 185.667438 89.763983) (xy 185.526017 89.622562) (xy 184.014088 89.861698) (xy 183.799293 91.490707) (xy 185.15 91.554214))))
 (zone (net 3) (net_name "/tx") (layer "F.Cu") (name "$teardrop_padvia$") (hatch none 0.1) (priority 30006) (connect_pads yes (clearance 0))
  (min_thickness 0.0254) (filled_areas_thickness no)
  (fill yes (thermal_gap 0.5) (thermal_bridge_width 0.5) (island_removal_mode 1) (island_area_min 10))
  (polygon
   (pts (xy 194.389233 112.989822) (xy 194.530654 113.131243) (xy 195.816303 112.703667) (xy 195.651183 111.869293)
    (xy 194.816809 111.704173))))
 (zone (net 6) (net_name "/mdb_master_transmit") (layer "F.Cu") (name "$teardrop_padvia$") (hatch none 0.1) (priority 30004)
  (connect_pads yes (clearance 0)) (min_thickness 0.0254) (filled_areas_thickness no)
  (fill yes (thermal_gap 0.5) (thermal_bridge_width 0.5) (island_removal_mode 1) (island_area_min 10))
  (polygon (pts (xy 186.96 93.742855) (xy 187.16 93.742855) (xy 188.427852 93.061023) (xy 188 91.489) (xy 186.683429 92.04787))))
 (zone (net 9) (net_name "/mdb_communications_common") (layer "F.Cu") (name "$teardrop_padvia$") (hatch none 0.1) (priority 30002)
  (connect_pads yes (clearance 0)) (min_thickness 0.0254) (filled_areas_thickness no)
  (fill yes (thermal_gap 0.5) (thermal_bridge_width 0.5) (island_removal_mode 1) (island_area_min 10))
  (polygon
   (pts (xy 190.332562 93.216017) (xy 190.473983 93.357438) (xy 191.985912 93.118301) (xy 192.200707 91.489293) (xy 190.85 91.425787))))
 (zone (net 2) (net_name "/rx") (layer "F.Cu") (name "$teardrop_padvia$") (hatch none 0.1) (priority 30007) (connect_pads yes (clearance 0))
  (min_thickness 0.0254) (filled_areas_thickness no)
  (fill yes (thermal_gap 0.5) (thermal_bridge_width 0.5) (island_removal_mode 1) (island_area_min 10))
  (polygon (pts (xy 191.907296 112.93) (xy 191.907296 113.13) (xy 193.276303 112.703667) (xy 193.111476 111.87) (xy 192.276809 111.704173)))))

